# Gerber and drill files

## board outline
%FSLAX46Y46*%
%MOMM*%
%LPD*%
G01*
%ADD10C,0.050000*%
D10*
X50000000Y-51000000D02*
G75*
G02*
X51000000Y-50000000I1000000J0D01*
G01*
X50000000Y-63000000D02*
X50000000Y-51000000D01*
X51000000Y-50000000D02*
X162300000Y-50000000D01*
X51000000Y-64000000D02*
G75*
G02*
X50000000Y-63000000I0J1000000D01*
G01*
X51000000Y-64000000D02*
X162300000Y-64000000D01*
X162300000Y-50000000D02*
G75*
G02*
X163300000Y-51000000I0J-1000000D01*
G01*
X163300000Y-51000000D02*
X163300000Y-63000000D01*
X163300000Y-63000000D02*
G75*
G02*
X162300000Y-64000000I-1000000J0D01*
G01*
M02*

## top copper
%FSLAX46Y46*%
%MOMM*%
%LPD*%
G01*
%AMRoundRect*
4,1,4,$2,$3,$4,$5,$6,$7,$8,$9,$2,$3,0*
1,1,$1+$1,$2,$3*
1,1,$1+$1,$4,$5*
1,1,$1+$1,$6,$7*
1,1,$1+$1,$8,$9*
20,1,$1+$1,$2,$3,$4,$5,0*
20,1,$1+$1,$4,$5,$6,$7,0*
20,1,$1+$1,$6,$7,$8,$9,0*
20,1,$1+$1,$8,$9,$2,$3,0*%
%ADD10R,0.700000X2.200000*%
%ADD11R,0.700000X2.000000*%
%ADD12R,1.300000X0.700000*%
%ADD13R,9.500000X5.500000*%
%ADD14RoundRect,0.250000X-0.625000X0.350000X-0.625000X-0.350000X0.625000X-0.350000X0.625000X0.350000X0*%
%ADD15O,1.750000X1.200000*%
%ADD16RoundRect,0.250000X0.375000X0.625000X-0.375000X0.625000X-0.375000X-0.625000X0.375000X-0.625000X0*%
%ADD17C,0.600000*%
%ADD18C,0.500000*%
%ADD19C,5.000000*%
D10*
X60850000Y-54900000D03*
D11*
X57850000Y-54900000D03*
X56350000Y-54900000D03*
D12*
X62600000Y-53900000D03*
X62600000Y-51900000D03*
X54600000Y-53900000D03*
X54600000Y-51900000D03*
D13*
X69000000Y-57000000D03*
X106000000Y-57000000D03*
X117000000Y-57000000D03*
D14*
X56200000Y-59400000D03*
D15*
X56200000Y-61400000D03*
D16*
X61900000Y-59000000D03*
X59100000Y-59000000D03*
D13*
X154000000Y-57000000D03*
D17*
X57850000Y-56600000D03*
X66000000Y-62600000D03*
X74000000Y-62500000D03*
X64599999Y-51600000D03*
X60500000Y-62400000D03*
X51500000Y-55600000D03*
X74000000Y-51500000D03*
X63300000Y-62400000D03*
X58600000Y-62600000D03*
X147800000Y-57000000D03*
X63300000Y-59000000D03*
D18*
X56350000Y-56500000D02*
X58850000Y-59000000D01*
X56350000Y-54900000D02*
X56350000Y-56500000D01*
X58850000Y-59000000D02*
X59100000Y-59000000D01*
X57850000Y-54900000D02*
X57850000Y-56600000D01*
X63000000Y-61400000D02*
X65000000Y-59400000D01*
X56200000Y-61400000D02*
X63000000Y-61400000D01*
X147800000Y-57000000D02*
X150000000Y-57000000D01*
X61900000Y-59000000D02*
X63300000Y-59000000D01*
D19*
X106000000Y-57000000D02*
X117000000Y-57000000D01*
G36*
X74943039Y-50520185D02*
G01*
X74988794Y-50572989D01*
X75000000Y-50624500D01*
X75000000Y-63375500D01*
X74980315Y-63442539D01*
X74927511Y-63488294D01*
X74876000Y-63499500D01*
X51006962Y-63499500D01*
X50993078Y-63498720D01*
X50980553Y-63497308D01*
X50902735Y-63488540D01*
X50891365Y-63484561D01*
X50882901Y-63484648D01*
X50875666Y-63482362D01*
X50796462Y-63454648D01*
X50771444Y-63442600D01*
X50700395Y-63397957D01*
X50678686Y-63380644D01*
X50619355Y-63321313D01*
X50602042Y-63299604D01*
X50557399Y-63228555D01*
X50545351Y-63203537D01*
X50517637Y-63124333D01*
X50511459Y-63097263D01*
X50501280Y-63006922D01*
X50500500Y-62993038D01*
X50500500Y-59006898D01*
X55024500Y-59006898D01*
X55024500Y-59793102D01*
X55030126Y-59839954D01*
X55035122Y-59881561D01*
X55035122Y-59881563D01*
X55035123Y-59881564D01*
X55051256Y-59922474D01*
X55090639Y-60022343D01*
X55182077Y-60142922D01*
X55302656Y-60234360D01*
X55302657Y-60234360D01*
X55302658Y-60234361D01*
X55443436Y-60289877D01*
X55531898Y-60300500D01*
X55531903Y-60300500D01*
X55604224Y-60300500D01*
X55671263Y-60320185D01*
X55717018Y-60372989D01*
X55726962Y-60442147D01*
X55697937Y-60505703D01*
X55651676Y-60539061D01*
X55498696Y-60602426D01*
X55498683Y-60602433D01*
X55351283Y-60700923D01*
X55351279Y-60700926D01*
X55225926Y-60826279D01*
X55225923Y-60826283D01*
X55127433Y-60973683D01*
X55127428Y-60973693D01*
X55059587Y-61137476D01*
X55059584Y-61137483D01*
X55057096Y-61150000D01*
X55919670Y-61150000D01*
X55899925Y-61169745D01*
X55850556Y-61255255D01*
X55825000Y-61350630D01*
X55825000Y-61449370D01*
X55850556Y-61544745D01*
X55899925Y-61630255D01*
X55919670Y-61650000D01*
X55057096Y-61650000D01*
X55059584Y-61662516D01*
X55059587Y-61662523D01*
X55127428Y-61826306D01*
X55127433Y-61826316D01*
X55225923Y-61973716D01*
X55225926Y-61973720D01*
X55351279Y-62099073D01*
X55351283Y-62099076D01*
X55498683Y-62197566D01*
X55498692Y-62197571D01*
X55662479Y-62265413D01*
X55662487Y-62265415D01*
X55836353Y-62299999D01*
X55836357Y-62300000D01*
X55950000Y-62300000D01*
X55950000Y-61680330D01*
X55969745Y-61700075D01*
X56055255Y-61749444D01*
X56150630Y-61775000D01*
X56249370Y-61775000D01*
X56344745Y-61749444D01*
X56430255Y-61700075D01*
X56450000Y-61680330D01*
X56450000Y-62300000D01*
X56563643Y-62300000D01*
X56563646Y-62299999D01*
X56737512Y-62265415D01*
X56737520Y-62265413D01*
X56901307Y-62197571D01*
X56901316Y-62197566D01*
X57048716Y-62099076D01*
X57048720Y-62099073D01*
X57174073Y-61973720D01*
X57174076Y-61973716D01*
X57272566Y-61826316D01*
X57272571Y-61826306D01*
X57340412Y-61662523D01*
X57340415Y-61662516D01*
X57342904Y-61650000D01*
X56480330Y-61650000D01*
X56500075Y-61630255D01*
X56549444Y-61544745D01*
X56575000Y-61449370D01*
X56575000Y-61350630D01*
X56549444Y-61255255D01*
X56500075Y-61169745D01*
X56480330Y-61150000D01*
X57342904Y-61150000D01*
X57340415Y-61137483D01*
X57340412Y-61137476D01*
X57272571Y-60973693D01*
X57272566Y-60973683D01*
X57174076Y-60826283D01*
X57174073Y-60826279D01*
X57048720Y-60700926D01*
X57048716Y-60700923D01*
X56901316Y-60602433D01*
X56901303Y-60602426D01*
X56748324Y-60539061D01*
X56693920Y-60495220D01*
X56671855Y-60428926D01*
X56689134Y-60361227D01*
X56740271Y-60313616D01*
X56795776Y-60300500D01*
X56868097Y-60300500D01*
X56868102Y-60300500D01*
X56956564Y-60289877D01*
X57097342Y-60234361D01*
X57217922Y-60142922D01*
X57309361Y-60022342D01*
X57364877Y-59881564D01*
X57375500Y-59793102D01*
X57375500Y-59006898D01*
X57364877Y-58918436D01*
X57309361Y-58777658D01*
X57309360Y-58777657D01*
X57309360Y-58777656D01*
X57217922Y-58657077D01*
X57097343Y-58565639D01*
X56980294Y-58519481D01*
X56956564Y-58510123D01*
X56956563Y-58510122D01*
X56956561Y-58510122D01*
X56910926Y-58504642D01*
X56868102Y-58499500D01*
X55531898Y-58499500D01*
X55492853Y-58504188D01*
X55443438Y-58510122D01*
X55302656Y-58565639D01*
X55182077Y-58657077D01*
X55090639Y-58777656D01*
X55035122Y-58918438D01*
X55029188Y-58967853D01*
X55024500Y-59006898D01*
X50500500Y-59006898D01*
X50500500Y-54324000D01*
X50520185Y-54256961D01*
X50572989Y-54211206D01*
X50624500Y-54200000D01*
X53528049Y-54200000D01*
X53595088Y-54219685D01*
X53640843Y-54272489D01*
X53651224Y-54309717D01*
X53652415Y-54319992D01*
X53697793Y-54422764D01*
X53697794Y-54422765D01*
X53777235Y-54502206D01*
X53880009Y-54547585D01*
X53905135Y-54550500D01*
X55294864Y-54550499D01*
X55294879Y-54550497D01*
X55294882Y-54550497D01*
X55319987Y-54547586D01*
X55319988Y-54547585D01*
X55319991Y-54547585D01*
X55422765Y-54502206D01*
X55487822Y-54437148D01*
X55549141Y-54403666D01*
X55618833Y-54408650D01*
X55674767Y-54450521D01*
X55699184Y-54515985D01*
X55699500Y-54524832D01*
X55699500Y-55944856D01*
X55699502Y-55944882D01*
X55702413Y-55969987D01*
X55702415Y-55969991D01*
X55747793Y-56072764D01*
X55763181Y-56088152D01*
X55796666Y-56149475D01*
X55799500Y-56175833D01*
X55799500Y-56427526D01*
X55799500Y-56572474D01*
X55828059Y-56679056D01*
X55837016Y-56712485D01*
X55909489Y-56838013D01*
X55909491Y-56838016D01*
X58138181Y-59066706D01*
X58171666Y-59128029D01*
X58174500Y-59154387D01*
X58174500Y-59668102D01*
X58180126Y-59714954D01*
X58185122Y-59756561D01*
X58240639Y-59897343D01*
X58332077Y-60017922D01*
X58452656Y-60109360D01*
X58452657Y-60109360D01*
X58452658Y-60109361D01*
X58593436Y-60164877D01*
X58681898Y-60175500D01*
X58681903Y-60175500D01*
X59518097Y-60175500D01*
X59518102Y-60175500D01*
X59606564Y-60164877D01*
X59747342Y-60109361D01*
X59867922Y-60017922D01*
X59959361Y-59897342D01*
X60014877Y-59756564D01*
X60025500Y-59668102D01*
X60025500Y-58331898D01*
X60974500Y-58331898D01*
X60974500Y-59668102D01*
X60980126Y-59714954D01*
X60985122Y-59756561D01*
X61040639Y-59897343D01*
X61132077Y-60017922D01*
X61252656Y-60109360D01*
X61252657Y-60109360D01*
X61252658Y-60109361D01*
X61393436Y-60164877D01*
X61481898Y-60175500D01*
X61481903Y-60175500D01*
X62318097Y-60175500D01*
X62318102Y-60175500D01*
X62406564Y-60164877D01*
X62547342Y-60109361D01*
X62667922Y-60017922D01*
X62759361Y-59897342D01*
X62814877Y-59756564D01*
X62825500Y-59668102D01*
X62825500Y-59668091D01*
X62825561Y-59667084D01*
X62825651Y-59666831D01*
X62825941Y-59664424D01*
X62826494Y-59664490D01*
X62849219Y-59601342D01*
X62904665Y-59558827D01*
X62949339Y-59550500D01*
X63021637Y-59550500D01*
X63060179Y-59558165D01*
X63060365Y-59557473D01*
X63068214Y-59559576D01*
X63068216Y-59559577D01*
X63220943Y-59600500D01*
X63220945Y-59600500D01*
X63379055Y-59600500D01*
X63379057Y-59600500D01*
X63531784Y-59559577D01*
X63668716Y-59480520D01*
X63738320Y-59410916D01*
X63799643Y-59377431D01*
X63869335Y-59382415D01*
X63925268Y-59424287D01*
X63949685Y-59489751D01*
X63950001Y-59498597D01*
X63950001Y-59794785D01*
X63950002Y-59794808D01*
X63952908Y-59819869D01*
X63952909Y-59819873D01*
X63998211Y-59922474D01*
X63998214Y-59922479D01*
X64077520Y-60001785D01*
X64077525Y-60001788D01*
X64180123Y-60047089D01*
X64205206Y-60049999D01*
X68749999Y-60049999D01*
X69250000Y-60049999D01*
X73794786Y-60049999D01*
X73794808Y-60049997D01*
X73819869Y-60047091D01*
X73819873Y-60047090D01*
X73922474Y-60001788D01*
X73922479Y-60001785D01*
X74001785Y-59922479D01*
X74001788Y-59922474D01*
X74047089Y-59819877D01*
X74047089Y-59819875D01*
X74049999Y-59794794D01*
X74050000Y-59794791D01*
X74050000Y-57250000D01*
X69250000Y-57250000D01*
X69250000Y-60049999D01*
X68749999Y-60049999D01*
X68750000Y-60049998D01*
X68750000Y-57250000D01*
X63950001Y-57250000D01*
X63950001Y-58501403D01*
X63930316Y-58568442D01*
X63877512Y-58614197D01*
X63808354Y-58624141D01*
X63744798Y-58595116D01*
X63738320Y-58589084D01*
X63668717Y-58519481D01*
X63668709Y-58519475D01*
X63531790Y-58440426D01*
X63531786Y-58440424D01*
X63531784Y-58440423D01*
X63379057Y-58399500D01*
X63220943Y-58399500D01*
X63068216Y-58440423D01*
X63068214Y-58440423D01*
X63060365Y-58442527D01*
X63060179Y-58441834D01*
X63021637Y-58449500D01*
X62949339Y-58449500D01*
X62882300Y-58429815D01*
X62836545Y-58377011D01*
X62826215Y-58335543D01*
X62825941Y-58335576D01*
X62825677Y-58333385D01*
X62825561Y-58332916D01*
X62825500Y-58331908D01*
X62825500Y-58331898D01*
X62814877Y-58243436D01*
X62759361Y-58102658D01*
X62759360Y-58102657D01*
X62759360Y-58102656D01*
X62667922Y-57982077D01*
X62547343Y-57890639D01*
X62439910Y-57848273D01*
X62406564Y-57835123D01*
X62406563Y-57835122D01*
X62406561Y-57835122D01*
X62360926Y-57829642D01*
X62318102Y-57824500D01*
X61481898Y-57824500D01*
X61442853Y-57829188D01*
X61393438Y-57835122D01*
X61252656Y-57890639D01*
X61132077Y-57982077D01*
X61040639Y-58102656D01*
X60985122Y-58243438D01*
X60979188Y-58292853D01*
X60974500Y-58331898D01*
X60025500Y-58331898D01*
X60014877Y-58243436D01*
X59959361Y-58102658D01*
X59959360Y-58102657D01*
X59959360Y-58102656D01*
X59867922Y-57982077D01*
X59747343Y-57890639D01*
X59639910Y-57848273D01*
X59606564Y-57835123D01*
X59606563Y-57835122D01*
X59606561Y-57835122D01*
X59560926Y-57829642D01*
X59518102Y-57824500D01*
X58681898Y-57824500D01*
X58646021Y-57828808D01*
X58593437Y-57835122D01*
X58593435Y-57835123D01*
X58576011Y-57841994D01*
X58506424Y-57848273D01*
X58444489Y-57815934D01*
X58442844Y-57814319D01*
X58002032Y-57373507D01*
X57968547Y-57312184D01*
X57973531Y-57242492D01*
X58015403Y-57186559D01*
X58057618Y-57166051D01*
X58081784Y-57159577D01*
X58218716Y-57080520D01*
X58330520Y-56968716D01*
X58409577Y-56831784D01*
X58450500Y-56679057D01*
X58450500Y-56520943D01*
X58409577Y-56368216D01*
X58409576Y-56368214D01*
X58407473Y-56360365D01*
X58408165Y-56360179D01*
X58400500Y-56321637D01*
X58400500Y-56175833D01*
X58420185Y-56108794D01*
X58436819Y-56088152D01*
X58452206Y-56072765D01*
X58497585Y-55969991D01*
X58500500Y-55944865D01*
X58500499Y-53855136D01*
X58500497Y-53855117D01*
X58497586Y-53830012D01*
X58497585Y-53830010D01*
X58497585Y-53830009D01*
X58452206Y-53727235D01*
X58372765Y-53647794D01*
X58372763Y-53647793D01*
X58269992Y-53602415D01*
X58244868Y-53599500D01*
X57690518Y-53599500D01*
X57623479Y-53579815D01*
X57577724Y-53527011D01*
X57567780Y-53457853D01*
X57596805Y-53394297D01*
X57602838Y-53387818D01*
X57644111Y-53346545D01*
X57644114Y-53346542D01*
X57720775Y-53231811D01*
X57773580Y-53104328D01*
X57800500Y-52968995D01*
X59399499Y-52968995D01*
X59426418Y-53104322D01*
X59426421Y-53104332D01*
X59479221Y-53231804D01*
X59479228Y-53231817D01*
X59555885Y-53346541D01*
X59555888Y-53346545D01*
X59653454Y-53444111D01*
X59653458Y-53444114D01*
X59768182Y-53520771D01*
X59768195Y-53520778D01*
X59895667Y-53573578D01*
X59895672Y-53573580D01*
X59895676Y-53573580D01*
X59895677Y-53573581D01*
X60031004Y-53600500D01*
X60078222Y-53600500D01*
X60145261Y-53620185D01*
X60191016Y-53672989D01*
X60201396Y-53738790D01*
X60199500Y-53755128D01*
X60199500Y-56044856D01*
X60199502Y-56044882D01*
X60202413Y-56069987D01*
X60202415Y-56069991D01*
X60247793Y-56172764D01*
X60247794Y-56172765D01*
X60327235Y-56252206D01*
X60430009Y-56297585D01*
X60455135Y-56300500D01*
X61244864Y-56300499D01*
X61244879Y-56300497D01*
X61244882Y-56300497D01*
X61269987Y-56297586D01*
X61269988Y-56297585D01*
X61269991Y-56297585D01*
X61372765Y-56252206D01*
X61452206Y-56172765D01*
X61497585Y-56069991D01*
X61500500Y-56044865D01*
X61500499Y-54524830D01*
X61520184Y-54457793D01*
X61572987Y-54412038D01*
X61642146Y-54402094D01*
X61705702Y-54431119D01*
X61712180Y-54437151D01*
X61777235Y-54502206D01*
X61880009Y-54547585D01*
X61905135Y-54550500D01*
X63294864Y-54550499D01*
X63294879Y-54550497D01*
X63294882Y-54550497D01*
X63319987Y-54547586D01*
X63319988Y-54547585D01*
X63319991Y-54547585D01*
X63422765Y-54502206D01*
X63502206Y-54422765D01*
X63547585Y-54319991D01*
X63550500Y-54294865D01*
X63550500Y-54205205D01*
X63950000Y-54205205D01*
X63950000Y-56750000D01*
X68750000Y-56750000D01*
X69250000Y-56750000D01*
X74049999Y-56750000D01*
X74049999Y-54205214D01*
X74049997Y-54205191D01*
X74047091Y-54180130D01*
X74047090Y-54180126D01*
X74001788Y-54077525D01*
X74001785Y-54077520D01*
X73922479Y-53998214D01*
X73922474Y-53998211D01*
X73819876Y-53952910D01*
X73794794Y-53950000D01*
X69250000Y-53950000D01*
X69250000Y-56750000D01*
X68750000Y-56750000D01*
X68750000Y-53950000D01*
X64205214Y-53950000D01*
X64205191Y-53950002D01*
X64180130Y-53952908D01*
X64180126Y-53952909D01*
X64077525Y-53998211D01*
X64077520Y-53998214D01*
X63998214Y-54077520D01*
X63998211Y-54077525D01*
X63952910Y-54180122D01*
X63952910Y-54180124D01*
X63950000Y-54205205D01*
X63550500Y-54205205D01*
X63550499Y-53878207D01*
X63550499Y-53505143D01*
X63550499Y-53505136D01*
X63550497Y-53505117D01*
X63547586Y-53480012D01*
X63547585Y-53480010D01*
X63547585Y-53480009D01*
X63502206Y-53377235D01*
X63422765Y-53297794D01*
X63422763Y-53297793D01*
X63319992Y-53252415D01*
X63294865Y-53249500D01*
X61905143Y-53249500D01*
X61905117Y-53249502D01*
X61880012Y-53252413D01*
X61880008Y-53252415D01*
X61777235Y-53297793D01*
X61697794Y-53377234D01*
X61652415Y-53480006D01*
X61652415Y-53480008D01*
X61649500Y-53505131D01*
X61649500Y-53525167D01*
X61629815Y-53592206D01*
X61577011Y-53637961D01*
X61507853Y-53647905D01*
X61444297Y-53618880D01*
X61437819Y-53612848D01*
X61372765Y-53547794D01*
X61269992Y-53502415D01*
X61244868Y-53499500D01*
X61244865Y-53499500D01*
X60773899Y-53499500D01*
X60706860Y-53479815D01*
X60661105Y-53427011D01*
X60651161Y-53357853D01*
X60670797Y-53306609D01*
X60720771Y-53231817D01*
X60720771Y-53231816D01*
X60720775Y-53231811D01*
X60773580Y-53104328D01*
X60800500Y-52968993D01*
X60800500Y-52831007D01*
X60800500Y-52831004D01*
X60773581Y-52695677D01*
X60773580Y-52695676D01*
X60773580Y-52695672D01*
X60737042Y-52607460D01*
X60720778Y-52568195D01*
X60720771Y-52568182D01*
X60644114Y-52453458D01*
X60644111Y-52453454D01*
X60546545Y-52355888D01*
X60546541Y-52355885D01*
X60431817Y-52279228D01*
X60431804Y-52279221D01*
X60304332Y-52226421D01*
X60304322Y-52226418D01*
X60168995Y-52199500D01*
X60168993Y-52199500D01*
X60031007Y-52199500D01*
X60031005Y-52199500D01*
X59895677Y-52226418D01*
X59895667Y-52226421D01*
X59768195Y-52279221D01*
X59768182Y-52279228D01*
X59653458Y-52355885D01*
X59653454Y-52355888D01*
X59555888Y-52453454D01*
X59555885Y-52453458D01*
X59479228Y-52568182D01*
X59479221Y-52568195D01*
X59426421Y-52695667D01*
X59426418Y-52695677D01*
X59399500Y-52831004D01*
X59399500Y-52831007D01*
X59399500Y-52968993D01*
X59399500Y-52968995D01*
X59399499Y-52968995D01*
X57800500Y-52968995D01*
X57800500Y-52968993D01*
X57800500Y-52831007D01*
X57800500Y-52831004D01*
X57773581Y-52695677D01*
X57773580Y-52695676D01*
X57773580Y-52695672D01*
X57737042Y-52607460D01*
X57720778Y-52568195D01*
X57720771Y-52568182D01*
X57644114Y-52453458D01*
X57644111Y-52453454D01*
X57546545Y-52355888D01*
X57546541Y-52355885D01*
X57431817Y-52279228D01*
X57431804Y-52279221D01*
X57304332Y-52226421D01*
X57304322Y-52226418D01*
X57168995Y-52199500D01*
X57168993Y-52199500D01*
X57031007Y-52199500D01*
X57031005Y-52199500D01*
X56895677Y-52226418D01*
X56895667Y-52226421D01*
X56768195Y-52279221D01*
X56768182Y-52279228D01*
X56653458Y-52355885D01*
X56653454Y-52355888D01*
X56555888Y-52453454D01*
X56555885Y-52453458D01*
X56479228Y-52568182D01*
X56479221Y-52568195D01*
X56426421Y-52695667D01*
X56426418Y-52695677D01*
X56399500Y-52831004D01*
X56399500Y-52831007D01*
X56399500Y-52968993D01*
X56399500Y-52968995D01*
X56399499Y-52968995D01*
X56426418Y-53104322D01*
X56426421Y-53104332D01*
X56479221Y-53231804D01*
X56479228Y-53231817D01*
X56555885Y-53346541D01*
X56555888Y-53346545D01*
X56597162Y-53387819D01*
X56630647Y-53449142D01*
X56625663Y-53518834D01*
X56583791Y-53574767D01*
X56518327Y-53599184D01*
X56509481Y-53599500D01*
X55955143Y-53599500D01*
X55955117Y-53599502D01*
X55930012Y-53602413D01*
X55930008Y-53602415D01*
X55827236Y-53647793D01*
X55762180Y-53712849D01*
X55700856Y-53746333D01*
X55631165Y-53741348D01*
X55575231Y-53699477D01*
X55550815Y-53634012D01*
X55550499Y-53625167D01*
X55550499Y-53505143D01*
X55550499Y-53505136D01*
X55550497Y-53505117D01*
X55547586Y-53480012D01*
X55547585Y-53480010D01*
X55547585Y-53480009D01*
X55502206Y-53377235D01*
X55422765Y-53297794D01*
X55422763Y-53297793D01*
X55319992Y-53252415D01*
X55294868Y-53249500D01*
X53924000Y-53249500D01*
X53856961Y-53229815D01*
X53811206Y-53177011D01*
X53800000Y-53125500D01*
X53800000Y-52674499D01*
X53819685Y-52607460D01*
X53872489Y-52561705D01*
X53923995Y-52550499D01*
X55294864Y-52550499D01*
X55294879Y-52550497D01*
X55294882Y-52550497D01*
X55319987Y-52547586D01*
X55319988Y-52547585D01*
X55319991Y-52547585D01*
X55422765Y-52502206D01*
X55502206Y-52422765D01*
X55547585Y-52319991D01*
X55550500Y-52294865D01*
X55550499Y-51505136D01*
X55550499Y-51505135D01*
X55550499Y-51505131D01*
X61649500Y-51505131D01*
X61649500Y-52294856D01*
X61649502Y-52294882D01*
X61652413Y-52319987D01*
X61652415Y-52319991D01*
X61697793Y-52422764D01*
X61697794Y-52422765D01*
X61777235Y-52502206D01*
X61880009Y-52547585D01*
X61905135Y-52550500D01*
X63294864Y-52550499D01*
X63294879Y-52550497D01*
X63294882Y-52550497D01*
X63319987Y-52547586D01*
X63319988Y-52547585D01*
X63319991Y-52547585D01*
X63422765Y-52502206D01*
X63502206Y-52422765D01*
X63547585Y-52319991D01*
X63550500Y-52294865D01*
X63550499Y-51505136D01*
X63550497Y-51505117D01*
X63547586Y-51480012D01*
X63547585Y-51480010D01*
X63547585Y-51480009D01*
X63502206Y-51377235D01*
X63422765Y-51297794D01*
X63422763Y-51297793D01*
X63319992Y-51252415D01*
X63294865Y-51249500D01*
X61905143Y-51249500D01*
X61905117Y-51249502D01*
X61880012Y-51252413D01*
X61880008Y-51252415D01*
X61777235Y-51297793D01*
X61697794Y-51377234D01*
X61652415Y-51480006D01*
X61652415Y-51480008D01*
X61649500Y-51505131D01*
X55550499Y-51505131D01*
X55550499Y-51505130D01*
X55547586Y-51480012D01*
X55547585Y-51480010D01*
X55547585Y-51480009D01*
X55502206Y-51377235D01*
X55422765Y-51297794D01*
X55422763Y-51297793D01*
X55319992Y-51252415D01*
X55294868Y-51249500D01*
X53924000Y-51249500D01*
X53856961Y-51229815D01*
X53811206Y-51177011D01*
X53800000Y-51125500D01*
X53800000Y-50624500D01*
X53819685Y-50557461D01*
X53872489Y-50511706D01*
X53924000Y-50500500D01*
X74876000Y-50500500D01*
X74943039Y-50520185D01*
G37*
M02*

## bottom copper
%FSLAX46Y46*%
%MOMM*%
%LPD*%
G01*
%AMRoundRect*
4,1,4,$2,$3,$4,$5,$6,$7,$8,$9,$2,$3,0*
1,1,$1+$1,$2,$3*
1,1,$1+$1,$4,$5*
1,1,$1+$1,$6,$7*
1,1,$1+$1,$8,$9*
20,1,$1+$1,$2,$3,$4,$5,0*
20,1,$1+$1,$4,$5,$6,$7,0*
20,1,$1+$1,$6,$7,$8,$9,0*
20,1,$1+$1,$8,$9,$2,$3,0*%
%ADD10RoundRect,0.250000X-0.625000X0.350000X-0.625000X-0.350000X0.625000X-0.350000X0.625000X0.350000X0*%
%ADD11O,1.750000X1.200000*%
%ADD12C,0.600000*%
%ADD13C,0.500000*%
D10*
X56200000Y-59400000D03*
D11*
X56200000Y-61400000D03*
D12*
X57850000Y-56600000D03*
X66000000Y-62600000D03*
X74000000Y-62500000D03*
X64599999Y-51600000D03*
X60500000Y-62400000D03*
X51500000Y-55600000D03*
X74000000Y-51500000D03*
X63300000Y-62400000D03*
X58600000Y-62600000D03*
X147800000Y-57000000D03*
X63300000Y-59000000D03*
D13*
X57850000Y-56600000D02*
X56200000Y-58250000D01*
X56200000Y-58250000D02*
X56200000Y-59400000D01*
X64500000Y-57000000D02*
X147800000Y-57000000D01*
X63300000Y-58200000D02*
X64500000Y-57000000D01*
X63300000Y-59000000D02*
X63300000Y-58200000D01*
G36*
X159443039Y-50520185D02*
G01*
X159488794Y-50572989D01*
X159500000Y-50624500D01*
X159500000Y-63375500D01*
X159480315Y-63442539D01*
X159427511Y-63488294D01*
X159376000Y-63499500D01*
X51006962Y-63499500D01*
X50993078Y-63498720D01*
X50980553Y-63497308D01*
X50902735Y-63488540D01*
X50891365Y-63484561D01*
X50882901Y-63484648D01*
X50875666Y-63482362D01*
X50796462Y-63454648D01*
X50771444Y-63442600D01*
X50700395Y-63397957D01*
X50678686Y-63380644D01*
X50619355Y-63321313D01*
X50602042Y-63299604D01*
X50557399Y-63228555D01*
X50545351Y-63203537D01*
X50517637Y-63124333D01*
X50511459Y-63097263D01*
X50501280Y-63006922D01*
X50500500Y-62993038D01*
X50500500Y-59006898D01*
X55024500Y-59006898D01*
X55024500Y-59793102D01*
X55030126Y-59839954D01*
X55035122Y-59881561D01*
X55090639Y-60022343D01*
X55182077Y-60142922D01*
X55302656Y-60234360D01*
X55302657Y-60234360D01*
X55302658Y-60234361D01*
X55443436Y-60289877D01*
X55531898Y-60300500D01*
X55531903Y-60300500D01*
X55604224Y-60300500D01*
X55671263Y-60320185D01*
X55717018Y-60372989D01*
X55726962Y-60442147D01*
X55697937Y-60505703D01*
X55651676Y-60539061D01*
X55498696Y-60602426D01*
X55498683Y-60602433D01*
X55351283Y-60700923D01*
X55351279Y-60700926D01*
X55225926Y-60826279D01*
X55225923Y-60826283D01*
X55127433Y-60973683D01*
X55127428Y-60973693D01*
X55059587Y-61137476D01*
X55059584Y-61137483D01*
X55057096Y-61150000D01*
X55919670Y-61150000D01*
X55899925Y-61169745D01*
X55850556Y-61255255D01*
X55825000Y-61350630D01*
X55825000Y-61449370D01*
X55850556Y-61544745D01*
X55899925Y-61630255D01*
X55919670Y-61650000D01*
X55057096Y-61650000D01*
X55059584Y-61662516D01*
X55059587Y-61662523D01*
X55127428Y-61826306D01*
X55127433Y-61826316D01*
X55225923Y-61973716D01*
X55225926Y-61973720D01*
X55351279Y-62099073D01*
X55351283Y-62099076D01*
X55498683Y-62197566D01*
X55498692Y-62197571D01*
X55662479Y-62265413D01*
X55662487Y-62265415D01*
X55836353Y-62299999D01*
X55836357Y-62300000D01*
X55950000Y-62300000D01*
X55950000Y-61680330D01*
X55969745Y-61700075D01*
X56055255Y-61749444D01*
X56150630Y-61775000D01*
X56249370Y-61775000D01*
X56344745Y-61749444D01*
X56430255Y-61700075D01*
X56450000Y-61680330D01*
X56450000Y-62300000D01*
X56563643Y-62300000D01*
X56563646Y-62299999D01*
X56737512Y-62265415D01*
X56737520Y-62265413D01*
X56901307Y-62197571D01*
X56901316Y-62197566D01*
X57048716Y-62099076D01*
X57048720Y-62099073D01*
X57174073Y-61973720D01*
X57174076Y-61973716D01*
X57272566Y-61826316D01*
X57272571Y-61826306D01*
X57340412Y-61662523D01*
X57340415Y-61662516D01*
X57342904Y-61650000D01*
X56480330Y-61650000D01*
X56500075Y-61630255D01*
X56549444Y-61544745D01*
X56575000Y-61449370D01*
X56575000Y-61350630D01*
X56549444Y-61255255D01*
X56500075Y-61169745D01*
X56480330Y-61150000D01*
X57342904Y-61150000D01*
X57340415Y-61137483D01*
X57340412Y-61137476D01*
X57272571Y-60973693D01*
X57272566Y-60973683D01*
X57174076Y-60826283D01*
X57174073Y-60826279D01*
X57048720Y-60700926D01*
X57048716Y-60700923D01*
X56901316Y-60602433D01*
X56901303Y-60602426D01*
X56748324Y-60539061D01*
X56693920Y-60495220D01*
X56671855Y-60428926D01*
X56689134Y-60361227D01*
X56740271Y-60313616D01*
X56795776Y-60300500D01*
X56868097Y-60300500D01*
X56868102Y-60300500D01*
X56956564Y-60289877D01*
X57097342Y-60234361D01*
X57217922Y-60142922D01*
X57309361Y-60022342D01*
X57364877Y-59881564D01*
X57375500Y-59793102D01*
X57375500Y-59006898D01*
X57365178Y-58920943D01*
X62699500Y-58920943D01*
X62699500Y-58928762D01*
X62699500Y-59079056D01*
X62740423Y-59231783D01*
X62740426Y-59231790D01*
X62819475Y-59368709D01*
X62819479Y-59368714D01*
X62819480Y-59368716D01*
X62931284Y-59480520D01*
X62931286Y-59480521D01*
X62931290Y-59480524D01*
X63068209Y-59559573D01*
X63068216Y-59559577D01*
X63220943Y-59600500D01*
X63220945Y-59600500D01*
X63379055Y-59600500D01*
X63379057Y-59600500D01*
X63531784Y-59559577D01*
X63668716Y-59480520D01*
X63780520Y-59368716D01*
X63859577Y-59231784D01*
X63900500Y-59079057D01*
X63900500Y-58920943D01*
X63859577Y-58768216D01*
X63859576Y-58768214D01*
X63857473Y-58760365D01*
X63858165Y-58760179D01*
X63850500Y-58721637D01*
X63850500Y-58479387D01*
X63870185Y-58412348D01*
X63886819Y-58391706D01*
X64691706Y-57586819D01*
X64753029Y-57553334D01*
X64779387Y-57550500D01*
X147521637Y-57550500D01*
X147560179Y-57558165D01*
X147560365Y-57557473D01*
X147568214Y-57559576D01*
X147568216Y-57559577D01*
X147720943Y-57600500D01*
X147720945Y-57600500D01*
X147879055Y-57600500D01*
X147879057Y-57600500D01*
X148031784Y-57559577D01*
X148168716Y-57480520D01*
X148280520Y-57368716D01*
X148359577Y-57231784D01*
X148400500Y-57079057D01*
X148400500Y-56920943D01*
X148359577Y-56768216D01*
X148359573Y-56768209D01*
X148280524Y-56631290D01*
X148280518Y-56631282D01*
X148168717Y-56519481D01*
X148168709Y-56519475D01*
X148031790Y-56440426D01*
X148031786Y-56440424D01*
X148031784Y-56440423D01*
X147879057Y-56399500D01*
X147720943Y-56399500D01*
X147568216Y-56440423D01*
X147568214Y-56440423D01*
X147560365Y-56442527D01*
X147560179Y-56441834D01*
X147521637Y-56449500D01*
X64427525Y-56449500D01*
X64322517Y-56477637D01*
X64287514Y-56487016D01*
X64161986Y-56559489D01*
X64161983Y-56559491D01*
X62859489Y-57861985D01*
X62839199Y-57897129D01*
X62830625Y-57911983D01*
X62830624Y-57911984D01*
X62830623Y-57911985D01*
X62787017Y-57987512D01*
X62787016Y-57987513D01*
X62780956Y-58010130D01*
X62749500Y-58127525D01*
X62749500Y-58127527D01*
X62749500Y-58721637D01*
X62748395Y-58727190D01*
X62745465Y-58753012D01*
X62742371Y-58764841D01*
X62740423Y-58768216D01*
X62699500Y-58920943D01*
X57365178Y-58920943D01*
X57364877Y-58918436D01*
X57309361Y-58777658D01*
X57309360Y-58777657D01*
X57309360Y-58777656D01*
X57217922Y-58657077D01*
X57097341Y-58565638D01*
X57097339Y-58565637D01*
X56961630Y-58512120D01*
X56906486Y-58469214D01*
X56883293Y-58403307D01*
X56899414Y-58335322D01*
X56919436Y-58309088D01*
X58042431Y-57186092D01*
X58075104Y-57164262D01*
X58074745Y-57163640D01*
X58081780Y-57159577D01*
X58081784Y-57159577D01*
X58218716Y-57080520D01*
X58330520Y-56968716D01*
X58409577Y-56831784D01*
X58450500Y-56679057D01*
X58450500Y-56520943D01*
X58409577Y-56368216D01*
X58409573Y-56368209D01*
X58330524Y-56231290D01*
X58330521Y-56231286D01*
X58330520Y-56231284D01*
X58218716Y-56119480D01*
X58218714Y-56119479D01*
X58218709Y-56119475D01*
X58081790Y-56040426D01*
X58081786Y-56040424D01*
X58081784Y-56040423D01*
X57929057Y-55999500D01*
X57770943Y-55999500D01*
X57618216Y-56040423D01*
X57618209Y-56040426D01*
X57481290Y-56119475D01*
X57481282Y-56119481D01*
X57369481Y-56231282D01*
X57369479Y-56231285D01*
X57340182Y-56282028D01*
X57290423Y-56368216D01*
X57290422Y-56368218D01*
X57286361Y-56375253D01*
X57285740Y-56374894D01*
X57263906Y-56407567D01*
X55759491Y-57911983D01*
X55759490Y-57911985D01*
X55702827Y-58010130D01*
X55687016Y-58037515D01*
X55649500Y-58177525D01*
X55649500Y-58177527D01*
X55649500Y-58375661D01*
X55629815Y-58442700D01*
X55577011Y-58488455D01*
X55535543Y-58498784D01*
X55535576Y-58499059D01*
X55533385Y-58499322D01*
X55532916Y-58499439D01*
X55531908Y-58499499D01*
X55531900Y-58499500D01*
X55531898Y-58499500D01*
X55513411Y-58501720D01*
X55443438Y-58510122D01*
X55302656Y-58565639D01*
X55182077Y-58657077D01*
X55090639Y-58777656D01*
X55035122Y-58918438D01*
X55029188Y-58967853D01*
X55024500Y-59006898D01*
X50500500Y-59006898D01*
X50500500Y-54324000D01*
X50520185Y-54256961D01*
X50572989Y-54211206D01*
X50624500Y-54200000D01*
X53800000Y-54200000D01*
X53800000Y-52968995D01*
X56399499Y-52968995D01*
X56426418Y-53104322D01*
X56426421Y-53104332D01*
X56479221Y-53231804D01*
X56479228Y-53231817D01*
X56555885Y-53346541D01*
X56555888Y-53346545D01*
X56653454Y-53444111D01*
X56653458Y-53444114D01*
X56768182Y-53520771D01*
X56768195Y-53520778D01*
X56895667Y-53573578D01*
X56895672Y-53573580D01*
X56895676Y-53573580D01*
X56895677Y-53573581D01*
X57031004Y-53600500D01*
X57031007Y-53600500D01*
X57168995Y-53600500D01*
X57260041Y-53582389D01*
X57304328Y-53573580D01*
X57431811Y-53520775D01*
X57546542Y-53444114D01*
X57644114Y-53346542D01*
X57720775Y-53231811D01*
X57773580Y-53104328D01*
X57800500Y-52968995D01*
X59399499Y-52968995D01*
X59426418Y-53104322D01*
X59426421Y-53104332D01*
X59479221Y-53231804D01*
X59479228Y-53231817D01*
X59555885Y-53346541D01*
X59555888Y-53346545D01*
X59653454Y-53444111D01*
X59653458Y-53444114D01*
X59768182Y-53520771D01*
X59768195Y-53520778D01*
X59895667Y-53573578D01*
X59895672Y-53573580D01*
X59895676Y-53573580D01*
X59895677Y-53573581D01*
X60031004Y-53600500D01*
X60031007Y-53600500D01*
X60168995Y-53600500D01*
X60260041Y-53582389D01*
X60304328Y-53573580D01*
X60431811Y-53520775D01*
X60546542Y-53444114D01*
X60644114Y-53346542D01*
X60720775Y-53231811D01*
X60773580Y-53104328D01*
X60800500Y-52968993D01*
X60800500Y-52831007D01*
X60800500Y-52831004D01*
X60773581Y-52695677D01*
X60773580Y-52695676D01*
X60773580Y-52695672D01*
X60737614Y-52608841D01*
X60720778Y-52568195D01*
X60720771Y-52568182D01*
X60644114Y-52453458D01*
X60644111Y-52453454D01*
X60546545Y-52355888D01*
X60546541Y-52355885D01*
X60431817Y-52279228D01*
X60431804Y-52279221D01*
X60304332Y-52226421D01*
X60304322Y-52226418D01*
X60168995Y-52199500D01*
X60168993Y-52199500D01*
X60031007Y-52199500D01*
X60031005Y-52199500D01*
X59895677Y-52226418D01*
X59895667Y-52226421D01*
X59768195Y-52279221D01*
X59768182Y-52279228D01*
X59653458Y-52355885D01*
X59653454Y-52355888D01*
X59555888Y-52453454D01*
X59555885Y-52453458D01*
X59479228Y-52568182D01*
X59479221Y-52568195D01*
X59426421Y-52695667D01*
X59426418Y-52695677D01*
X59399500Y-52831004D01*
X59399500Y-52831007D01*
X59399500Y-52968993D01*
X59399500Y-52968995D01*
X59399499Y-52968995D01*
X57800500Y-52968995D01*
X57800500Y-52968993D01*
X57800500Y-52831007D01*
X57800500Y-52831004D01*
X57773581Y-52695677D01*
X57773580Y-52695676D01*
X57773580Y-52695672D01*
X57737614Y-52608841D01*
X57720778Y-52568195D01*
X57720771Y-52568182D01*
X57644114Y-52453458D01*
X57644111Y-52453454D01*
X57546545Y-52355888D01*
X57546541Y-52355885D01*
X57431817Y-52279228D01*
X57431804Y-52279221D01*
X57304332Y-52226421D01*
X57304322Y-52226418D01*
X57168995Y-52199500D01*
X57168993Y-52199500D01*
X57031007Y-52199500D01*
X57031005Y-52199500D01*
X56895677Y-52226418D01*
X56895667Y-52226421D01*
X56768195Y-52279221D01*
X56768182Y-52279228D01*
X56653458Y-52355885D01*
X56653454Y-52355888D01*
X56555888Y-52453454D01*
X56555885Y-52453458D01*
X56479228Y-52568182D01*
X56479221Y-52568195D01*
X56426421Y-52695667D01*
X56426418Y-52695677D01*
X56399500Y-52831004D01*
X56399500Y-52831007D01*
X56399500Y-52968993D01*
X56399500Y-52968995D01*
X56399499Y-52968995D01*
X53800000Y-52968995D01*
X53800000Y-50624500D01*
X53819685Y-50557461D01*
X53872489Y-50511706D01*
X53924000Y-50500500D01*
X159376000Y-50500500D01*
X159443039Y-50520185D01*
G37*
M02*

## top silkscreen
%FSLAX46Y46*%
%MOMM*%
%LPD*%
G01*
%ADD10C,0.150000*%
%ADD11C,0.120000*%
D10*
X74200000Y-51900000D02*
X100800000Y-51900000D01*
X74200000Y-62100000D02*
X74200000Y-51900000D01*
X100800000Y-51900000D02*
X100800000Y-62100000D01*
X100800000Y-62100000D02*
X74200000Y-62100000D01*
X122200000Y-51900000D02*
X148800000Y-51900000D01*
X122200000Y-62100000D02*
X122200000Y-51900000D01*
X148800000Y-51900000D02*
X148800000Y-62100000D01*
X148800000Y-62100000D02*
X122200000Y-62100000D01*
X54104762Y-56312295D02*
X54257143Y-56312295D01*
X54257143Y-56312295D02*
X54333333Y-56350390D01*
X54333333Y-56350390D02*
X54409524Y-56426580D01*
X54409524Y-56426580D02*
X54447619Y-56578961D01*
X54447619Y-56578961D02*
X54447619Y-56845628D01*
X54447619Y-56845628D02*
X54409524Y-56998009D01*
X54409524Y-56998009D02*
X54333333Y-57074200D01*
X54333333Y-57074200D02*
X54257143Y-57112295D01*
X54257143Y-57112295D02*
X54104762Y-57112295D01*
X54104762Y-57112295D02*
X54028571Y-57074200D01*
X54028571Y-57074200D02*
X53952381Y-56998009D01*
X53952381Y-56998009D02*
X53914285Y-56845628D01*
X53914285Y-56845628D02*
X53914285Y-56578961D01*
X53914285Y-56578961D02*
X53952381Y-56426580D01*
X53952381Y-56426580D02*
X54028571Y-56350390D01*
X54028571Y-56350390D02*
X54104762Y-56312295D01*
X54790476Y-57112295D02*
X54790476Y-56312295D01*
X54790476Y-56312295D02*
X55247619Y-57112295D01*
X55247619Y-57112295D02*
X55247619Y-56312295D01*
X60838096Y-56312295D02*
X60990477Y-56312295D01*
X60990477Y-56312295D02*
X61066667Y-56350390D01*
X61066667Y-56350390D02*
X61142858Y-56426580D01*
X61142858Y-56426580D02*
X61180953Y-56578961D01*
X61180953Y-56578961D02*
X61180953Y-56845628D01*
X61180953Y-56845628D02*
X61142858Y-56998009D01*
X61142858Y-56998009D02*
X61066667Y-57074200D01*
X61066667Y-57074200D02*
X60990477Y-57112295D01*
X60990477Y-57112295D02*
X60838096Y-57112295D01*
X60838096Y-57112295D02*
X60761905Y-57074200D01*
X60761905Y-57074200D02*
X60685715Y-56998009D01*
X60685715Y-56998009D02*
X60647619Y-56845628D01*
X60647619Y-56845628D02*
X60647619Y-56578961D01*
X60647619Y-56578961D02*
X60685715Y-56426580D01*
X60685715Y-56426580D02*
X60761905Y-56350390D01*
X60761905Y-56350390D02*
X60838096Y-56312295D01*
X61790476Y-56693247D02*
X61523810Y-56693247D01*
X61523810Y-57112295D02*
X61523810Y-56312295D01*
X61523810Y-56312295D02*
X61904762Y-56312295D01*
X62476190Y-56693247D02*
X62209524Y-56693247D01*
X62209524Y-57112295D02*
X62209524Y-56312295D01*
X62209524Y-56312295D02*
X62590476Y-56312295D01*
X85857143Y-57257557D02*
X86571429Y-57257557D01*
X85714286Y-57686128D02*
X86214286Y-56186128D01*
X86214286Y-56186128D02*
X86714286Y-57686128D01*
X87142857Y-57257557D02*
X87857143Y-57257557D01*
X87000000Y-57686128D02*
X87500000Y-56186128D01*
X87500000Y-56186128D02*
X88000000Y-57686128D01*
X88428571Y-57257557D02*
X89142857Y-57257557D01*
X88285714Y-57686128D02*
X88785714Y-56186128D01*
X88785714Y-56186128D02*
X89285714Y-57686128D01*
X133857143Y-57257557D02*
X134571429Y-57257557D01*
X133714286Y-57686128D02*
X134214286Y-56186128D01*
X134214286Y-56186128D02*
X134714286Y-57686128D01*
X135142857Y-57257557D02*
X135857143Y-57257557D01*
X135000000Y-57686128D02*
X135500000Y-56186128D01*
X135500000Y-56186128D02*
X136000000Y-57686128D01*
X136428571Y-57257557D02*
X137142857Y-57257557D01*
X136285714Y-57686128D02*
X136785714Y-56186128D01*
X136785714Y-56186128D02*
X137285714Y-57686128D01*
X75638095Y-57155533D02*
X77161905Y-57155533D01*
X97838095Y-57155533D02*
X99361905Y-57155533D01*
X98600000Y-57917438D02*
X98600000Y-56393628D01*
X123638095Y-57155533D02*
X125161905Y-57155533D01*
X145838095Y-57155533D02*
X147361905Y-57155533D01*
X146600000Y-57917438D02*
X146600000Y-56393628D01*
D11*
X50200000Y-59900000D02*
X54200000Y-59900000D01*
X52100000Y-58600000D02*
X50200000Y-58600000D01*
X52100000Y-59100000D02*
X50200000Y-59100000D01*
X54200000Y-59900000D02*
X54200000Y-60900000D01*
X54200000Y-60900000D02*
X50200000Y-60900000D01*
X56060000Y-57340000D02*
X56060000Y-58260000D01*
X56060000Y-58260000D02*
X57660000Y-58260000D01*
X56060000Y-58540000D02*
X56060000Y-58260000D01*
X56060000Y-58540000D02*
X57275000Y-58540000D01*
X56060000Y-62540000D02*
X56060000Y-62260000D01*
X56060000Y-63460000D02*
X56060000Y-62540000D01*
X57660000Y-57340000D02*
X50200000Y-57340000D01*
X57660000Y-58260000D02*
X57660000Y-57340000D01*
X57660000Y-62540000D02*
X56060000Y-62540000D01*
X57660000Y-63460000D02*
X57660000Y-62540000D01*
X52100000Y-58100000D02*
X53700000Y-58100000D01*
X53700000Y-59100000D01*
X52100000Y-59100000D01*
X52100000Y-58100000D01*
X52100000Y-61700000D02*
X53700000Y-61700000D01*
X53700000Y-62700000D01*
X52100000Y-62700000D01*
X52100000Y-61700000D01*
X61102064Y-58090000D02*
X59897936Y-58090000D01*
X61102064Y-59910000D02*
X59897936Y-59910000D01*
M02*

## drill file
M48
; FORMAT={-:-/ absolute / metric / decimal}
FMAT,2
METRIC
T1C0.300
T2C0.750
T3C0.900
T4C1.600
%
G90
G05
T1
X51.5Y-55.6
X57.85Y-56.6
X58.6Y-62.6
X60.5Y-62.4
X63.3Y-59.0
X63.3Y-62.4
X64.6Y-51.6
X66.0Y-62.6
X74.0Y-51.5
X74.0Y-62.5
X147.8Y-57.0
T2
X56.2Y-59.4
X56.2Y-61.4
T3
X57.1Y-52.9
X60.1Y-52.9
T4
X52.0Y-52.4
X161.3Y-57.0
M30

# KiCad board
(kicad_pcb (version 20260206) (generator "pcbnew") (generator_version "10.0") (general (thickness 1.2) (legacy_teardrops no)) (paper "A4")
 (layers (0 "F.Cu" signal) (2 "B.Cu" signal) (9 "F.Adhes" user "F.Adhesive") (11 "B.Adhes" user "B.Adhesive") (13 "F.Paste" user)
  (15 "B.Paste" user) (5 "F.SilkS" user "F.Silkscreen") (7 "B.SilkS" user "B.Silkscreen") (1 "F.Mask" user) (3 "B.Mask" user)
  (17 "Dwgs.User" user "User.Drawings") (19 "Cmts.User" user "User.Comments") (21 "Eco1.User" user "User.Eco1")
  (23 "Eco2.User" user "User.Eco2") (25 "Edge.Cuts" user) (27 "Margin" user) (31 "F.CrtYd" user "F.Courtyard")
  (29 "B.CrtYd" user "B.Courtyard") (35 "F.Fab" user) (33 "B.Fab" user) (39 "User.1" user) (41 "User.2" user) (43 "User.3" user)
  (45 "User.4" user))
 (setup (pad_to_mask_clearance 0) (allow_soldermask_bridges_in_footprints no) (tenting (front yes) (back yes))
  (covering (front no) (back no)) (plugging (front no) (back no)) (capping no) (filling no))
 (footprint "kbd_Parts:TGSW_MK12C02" (layer "F.Cu") (at 58.6 52.9 180)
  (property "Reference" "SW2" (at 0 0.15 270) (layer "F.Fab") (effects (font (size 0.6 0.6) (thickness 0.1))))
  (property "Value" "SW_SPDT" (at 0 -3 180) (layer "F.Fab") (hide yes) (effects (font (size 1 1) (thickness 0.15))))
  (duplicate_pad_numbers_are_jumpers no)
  (pad "" np_thru_hole circle (at -1.5 0 180) (size 0.9 0.9) (drill 0.9) (layers "*.Cu" "*.Mask"))
  (pad "" np_thru_hole circle (at 1.5 0 180) (size 0.9 0.9) (drill 0.9) (layers "*.Cu" "*.Mask"))
  (pad "1" smd rect (at -2.25 -2 180) (size 0.7 2.2) (layers "F.Cu" "F.Mask" "F.Paste") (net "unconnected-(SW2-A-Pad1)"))
  (pad "2" smd rect (at 0.75 -2 180) (size 0.7 2) (layers "F.Cu" "F.Mask" "F.Paste") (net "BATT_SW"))
  (pad "3" smd rect (at 2.25 -2 180) (size 0.7 2) (layers "F.Cu" "F.Mask" "F.Paste") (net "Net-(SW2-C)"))
  (pad "4" smd rect (at -4 -1 90) (size 0.7 1.3) (layers "F.Cu" "F.Mask" "F.Paste"))
  (pad "4" smd rect (at -4 1 90) (size 0.7 1.3) (layers "F.Cu" "F.Mask" "F.Paste"))
  (pad "4" smd rect (at 4 -1 90) (size 0.7 1.3) (layers "F.Cu" "F.Mask" "F.Paste"))
  (pad "4" smd rect (at 4 1 90) (size 0.7 1.3) (layers "F.Cu" "F.Mask" "F.Paste")))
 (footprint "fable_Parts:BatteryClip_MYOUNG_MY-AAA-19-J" (layer "F.Cu") (at 69 57)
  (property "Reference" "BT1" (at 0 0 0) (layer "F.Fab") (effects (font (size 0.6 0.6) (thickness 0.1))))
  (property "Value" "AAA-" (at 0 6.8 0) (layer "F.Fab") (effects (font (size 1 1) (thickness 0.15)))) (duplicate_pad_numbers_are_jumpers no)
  (pad "1" smd rect (at 0 0) (size 9.5 5.5) (layers "F.Cu" "F.Mask" "F.Paste") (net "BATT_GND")))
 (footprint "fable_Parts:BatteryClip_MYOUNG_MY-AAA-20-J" (layer "F.Cu") (at 106 57 180)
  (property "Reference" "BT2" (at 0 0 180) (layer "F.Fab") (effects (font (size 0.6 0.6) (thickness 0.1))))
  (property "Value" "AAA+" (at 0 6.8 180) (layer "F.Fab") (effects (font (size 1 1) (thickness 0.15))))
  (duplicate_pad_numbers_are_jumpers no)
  (pad "1" smd rect (at 0 0 180) (size 9.5 5.5) (layers "F.Cu" "F.Mask" "F.Paste") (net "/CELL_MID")))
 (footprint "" (layer "F.Cu") (at 52 52.4)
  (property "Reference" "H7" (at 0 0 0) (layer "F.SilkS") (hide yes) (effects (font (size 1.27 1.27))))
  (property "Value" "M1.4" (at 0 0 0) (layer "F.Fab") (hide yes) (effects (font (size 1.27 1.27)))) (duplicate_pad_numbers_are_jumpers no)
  (pad "" np_thru_hole circle (at 0 0) (size 1.6 1.6) (drill 1.6) (layers "*.Cu")))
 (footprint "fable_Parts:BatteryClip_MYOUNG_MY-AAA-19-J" (layer "F.Cu") (at 117 57)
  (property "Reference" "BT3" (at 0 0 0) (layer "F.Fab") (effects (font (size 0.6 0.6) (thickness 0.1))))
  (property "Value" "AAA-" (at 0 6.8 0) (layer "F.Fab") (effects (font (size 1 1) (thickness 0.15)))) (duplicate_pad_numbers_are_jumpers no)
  (pad "1" smd rect (at 0 0) (size 9.5 5.5) (layers "F.Cu" "F.Mask" "F.Paste") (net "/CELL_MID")))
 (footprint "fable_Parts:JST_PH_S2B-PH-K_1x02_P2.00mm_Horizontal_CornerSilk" (layer "F.Cu") (at 56.2 59.4 -90)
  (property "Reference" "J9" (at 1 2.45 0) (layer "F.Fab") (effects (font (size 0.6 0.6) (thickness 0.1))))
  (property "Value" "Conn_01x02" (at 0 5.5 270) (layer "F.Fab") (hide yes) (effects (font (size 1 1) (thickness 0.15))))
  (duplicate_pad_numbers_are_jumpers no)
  (fp_line (start 0.5 6) (end 0.5 2) (stroke (width 0.12) (type solid)) (layer "F.SilkS"))
  (fp_line (start -0.8 4.1) (end -0.8 6) (stroke (width 0.12) (type solid)) (layer "F.SilkS"))
  (fp_line (start -0.3 4.1) (end -0.3 6) (stroke (width 0.12) (type solid)) (layer "F.SilkS"))
  (fp_line (start 0.5 2) (end 1.5 2) (stroke (width 0.12) (type solid)) (layer "F.SilkS"))
  (fp_line (start 1.5 2) (end 1.5 6) (stroke (width 0.12) (type solid)) (layer "F.SilkS"))
  (fp_line (start -2.06 0.14) (end -1.14 0.14) (stroke (width 0.12) (type solid)) (layer "F.SilkS"))
  (fp_line (start -1.14 0.14) (end -1.14 -1.46) (stroke (width 0.12) (type solid)) (layer "F.SilkS"))
  (fp_line (start -0.86 0.14) (end -1.14 0.14) (stroke (width 0.12) (type solid)) (layer "F.SilkS"))
  (fp_line (start -0.86 0.14) (end -0.86 -1.075) (stroke (width 0.12) (type solid)) (layer "F.SilkS"))
  (fp_line (start 3.14 0.14) (end 2.86 0.14) (stroke (width 0.12) (type solid)) (layer "F.SilkS"))
  (fp_line (start 4.06 0.14) (end 3.14 0.14) (stroke (width 0.12) (type solid)) (layer "F.SilkS"))
  (fp_line (start -2.06 -1.46) (end -2.06 6) (stroke (width 0.12) (type solid)) (layer "F.SilkS"))
  (fp_line (start -1.14 -1.46) (end -2.06 -1.46) (stroke (width 0.12) (type solid)) (layer "F.SilkS"))
  (fp_line (start 3.14 -1.46) (end 3.14 0.14) (stroke (width 0.12) (type solid)) (layer "F.SilkS"))
  (fp_line (start 4.06 -1.46) (end 3.14 -1.46) (stroke (width 0.12) (type solid)) (layer "F.SilkS"))
  (fp_rect (start -1.3 2.5) (end -0.3 4.1) (stroke (width 0.12) (type solid)) (fill no) (layer "F.SilkS"))
  (fp_rect (start 2.3 2.5) (end 3.3 4.1) (stroke (width 0.12) (type solid)) (fill no) (layer "F.SilkS"))
  (pad "1" thru_hole roundrect (at 0 0 270) (size 1.2 1.75) (drill 0.75) (layers "*.Cu" "*.Mask") (remove_unused_layers no)
   (roundrect_rratio 0.208333) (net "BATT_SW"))
  (pad "2" thru_hole oval (at 2 0 270) (size 1.2 1.75) (drill 0.75) (layers "*.Cu" "*.Mask") (remove_unused_layers no) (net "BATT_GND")))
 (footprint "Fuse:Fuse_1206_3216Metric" (layer "F.Cu") (at 60.5 59 180)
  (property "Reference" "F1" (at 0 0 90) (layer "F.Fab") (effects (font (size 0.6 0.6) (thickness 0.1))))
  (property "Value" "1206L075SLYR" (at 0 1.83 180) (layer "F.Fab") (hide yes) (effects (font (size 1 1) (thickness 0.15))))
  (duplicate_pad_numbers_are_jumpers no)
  (fp_line (start -0.602064 0.91) (end 0.602064 0.91) (stroke (width 0.12) (type solid)) (layer "F.SilkS"))
  (fp_line (start -0.602064 -0.91) (end 0.602064 -0.91) (stroke (width 0.12) (type solid)) (layer "F.SilkS"))
  (pad "1" smd roundrect (at -1.4 0 180) (size 1.25 1.75) (layers "F.Cu" "F.Mask" "F.Paste") (roundrect_rratio 0.2) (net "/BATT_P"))
  (pad "2" smd roundrect (at 1.4 0 180) (size 1.25 1.75) (layers "F.Cu" "F.Mask" "F.Paste") (roundrect_rratio 0.2) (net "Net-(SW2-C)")))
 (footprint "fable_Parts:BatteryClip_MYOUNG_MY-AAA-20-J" (layer "F.Cu") (at 154 57 180)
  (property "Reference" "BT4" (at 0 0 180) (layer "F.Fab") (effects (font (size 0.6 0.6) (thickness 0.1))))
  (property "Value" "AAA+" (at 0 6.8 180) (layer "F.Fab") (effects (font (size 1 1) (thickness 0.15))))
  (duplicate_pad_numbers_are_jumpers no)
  (pad "1" smd rect (at 0 0 180) (size 9.5 5.5) (layers "F.Cu" "F.Mask" "F.Paste") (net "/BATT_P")))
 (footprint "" (layer "F.Cu") (at 161.3 57)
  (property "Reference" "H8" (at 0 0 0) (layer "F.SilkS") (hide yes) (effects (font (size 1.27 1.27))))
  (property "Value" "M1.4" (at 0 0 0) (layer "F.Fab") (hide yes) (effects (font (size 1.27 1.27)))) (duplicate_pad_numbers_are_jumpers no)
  (pad "" np_thru_hole circle (at 0 0) (size 1.6 1.6) (drill 1.6) (layers "*.Cu")))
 (gr_line (start 74.2 51.9) (end 100.8 51.9) (stroke (width 0.15) (type default)) (layer "F.SilkS"))
 (gr_line (start 74.2 62.1) (end 74.2 51.9) (stroke (width 0.15) (type default)) (layer "F.SilkS"))
 (gr_line (start 100.8 51.9) (end 100.8 62.1) (stroke (width 0.15) (type default)) (layer "F.SilkS"))
 (gr_line (start 100.8 62.1) (end 74.2 62.1) (stroke (width 0.15) (type default)) (layer "F.SilkS"))
 (gr_line (start 122.2 51.9) (end 148.8 51.9) (stroke (width 0.15) (type default)) (layer "F.SilkS"))
 (gr_line (start 122.2 62.1) (end 122.2 51.9) (stroke (width 0.15) (type default)) (layer "F.SilkS"))
 (gr_line (start 148.8 51.9) (end 148.8 62.1) (stroke (width 0.15) (type default)) (layer "F.SilkS"))
 (gr_line (start 148.8 62.1) (end 122.2 62.1) (stroke (width 0.15) (type default)) (layer "F.SilkS"))
 (gr_arc (start 50 51) (mid 50.292893 50.292893) (end 51 50) (stroke (width 0.05) (type default)) (layer "Edge.Cuts"))
 (gr_line (start 50 63) (end 50 51) (stroke (width 0.05) (type default)) (layer "Edge.Cuts"))
 (gr_line (start 51 50) (end 162.3 50) (stroke (width 0.05) (type default)) (layer "Edge.Cuts"))
 (gr_arc (start 51 64) (mid 50.292893 63.707106) (end 50 63) (stroke (width 0.05) (type default)) (layer "Edge.Cuts"))
 (gr_line (start 51 64) (end 162.3 64) (stroke (width 0.05) (type default)) (layer "Edge.Cuts"))
 (gr_arc (start 162.3 50) (mid 163.007106 50.292893) (end 163.3 51) (stroke (width 0.05) (type default)) (layer "Edge.Cuts"))
 (gr_line (start 163.3 51) (end 163.3 63) (stroke (width 0.05) (type default)) (layer "Edge.Cuts"))
 (gr_arc (start 163.3 63) (mid 163.007106 63.707106) (end 162.3 64) (stroke (width 0.05) (type default)) (layer "Edge.Cuts"))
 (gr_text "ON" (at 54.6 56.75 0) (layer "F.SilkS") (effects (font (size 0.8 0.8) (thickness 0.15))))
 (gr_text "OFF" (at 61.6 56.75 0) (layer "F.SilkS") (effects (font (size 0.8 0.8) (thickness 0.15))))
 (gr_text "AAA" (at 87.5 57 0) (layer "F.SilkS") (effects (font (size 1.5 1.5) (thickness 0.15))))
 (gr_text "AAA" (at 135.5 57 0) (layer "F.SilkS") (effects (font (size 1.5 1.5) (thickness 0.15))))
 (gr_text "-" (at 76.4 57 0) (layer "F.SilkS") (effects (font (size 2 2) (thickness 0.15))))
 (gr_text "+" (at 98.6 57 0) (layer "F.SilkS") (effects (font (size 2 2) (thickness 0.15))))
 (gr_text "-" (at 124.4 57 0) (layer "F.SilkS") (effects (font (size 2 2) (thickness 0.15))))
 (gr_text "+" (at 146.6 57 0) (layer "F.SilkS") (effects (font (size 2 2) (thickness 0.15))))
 (segment (start 56.35 56.5) (end 58.85 59) (width 0.5) (layer "F.Cu") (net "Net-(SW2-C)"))
 (segment (start 56.35 54.9) (end 56.35 56.5) (width 0.5) (layer "F.Cu") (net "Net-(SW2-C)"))
 (segment (start 58.85 59) (end 59.1 59) (width 0.5) (layer "F.Cu") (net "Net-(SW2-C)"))
 (segment (start 57.85 54.9) (end 57.85 56.6) (width 0.5) (layer "F.Cu") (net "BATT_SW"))
 (via (at 57.85 56.6) (size 0.6) (drill 0.3) (layers "F.Cu" "B.Cu") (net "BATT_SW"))
 (segment (start 57.85 56.6) (end 56.2 58.25) (width 0.5) (layer "B.Cu") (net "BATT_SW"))
 (segment (start 56.2 58.25) (end 56.2 59.4) (width 0.5) (layer "B.Cu") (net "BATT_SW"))
 (segment (start 63 61.4) (end 65 59.4) (width 0.5) (layer "F.Cu") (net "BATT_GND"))
 (segment (start 56.2 61.4) (end 63 61.4) (width 0.5) (layer "F.Cu") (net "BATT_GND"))
 (via (at 66 62.6) (size 0.6) (drill 0.3) (layers "F.Cu" "B.Cu") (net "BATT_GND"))
 (via (at 74 62.5) (size 0.6) (drill 0.3) (layers "F.Cu" "B.Cu") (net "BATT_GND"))
 (via (at 64.599999 51.6) (size 0.6) (drill 0.3) (layers "F.Cu" "B.Cu") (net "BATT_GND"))
 (via (at 60.5 62.4) (size 0.6) (drill 0.3) (layers "F.Cu" "B.Cu") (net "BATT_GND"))
 (via (at 51.5 55.6) (size 0.6) (drill 0.3) (layers "F.Cu" "B.Cu") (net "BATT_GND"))
 (via (at 74 51.5) (size 0.6) (drill 0.3) (layers "F.Cu" "B.Cu") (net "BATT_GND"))
 (via (at 63.3 62.4) (size 0.6) (drill 0.3) (layers "F.Cu" "B.Cu") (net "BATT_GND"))
 (via (at 58.6 62.6) (size 0.6) (drill 0.3) (layers "F.Cu" "B.Cu") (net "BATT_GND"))
 (segment (start 147.8 57) (end 150 57) (width 0.5) (layer "F.Cu") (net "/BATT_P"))
 (segment (start 61.9 59) (end 63.3 59) (width 0.5) (layer "F.Cu") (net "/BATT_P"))
 (via (at 147.8 57) (size 0.6) (drill 0.3) (layers "F.Cu" "B.Cu") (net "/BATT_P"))
 (via (at 63.3 59) (size 0.6) (drill 0.3) (layers "F.Cu" "B.Cu") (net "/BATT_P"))
 (segment (start 64.5 57) (end 147.8 57) (width 0.5) (layer "B.Cu") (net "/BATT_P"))
 (segment (start 63.3 58.2) (end 64.5 57) (width 0.5) (layer "B.Cu") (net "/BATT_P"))
 (segment (start 63.3 59) (end 63.3 58.2) (width 0.5) (layer "B.Cu") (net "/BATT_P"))
 (segment (start 106 57) (end 117 57) (width 5) (layer "F.Cu") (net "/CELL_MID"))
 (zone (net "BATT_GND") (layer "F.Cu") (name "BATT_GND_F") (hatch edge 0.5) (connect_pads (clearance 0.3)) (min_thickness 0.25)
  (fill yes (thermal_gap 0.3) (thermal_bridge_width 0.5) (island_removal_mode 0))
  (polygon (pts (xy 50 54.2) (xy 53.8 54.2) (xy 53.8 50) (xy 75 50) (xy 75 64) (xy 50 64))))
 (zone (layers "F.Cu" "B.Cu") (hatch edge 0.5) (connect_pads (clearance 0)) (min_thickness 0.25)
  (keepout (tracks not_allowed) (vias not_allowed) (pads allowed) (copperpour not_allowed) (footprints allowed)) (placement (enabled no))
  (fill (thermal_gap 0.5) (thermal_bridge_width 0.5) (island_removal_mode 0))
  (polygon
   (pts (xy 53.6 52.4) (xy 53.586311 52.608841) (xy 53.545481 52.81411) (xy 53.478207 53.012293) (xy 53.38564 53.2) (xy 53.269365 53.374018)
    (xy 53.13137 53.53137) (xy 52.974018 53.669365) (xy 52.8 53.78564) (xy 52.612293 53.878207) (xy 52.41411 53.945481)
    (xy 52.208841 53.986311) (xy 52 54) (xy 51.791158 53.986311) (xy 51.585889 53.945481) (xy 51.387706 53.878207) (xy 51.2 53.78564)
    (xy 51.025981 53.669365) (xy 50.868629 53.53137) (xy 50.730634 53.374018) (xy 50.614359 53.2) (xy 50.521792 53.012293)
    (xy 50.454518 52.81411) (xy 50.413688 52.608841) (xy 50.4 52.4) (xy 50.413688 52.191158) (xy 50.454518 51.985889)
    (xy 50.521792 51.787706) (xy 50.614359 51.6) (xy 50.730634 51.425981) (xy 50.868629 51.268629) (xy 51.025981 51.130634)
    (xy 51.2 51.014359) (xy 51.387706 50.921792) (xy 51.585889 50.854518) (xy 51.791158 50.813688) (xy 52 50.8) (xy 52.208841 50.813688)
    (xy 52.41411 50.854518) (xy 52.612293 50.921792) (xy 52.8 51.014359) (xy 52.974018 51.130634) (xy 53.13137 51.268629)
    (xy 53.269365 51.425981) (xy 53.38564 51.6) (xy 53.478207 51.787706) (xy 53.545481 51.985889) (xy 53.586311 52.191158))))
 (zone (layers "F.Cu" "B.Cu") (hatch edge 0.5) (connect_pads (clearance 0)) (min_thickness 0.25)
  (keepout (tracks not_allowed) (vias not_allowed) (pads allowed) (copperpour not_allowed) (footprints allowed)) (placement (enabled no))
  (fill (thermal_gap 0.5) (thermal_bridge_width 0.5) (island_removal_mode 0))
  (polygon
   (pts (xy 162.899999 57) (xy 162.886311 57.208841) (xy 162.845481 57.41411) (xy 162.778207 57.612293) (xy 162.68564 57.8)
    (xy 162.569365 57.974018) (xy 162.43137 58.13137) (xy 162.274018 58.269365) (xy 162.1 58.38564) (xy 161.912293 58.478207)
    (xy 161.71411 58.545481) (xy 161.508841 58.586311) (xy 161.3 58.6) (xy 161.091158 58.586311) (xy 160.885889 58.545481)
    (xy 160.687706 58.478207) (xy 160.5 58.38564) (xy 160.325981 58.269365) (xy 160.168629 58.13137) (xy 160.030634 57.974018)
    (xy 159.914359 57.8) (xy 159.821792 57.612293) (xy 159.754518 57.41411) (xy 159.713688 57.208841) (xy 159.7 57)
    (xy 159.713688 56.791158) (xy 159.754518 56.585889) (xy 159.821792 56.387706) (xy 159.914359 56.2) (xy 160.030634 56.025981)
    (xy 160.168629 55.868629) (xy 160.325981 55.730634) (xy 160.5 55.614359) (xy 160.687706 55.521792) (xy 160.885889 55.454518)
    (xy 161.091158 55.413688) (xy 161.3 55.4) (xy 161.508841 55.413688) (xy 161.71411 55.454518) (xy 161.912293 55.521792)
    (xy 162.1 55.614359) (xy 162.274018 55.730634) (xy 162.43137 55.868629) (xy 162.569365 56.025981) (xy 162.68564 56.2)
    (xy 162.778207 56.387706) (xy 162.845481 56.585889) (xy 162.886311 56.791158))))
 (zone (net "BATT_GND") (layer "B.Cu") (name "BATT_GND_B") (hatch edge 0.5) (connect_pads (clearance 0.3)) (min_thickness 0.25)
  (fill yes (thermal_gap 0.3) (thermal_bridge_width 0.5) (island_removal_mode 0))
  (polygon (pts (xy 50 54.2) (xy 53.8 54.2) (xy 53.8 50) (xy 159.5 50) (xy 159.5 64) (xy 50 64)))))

